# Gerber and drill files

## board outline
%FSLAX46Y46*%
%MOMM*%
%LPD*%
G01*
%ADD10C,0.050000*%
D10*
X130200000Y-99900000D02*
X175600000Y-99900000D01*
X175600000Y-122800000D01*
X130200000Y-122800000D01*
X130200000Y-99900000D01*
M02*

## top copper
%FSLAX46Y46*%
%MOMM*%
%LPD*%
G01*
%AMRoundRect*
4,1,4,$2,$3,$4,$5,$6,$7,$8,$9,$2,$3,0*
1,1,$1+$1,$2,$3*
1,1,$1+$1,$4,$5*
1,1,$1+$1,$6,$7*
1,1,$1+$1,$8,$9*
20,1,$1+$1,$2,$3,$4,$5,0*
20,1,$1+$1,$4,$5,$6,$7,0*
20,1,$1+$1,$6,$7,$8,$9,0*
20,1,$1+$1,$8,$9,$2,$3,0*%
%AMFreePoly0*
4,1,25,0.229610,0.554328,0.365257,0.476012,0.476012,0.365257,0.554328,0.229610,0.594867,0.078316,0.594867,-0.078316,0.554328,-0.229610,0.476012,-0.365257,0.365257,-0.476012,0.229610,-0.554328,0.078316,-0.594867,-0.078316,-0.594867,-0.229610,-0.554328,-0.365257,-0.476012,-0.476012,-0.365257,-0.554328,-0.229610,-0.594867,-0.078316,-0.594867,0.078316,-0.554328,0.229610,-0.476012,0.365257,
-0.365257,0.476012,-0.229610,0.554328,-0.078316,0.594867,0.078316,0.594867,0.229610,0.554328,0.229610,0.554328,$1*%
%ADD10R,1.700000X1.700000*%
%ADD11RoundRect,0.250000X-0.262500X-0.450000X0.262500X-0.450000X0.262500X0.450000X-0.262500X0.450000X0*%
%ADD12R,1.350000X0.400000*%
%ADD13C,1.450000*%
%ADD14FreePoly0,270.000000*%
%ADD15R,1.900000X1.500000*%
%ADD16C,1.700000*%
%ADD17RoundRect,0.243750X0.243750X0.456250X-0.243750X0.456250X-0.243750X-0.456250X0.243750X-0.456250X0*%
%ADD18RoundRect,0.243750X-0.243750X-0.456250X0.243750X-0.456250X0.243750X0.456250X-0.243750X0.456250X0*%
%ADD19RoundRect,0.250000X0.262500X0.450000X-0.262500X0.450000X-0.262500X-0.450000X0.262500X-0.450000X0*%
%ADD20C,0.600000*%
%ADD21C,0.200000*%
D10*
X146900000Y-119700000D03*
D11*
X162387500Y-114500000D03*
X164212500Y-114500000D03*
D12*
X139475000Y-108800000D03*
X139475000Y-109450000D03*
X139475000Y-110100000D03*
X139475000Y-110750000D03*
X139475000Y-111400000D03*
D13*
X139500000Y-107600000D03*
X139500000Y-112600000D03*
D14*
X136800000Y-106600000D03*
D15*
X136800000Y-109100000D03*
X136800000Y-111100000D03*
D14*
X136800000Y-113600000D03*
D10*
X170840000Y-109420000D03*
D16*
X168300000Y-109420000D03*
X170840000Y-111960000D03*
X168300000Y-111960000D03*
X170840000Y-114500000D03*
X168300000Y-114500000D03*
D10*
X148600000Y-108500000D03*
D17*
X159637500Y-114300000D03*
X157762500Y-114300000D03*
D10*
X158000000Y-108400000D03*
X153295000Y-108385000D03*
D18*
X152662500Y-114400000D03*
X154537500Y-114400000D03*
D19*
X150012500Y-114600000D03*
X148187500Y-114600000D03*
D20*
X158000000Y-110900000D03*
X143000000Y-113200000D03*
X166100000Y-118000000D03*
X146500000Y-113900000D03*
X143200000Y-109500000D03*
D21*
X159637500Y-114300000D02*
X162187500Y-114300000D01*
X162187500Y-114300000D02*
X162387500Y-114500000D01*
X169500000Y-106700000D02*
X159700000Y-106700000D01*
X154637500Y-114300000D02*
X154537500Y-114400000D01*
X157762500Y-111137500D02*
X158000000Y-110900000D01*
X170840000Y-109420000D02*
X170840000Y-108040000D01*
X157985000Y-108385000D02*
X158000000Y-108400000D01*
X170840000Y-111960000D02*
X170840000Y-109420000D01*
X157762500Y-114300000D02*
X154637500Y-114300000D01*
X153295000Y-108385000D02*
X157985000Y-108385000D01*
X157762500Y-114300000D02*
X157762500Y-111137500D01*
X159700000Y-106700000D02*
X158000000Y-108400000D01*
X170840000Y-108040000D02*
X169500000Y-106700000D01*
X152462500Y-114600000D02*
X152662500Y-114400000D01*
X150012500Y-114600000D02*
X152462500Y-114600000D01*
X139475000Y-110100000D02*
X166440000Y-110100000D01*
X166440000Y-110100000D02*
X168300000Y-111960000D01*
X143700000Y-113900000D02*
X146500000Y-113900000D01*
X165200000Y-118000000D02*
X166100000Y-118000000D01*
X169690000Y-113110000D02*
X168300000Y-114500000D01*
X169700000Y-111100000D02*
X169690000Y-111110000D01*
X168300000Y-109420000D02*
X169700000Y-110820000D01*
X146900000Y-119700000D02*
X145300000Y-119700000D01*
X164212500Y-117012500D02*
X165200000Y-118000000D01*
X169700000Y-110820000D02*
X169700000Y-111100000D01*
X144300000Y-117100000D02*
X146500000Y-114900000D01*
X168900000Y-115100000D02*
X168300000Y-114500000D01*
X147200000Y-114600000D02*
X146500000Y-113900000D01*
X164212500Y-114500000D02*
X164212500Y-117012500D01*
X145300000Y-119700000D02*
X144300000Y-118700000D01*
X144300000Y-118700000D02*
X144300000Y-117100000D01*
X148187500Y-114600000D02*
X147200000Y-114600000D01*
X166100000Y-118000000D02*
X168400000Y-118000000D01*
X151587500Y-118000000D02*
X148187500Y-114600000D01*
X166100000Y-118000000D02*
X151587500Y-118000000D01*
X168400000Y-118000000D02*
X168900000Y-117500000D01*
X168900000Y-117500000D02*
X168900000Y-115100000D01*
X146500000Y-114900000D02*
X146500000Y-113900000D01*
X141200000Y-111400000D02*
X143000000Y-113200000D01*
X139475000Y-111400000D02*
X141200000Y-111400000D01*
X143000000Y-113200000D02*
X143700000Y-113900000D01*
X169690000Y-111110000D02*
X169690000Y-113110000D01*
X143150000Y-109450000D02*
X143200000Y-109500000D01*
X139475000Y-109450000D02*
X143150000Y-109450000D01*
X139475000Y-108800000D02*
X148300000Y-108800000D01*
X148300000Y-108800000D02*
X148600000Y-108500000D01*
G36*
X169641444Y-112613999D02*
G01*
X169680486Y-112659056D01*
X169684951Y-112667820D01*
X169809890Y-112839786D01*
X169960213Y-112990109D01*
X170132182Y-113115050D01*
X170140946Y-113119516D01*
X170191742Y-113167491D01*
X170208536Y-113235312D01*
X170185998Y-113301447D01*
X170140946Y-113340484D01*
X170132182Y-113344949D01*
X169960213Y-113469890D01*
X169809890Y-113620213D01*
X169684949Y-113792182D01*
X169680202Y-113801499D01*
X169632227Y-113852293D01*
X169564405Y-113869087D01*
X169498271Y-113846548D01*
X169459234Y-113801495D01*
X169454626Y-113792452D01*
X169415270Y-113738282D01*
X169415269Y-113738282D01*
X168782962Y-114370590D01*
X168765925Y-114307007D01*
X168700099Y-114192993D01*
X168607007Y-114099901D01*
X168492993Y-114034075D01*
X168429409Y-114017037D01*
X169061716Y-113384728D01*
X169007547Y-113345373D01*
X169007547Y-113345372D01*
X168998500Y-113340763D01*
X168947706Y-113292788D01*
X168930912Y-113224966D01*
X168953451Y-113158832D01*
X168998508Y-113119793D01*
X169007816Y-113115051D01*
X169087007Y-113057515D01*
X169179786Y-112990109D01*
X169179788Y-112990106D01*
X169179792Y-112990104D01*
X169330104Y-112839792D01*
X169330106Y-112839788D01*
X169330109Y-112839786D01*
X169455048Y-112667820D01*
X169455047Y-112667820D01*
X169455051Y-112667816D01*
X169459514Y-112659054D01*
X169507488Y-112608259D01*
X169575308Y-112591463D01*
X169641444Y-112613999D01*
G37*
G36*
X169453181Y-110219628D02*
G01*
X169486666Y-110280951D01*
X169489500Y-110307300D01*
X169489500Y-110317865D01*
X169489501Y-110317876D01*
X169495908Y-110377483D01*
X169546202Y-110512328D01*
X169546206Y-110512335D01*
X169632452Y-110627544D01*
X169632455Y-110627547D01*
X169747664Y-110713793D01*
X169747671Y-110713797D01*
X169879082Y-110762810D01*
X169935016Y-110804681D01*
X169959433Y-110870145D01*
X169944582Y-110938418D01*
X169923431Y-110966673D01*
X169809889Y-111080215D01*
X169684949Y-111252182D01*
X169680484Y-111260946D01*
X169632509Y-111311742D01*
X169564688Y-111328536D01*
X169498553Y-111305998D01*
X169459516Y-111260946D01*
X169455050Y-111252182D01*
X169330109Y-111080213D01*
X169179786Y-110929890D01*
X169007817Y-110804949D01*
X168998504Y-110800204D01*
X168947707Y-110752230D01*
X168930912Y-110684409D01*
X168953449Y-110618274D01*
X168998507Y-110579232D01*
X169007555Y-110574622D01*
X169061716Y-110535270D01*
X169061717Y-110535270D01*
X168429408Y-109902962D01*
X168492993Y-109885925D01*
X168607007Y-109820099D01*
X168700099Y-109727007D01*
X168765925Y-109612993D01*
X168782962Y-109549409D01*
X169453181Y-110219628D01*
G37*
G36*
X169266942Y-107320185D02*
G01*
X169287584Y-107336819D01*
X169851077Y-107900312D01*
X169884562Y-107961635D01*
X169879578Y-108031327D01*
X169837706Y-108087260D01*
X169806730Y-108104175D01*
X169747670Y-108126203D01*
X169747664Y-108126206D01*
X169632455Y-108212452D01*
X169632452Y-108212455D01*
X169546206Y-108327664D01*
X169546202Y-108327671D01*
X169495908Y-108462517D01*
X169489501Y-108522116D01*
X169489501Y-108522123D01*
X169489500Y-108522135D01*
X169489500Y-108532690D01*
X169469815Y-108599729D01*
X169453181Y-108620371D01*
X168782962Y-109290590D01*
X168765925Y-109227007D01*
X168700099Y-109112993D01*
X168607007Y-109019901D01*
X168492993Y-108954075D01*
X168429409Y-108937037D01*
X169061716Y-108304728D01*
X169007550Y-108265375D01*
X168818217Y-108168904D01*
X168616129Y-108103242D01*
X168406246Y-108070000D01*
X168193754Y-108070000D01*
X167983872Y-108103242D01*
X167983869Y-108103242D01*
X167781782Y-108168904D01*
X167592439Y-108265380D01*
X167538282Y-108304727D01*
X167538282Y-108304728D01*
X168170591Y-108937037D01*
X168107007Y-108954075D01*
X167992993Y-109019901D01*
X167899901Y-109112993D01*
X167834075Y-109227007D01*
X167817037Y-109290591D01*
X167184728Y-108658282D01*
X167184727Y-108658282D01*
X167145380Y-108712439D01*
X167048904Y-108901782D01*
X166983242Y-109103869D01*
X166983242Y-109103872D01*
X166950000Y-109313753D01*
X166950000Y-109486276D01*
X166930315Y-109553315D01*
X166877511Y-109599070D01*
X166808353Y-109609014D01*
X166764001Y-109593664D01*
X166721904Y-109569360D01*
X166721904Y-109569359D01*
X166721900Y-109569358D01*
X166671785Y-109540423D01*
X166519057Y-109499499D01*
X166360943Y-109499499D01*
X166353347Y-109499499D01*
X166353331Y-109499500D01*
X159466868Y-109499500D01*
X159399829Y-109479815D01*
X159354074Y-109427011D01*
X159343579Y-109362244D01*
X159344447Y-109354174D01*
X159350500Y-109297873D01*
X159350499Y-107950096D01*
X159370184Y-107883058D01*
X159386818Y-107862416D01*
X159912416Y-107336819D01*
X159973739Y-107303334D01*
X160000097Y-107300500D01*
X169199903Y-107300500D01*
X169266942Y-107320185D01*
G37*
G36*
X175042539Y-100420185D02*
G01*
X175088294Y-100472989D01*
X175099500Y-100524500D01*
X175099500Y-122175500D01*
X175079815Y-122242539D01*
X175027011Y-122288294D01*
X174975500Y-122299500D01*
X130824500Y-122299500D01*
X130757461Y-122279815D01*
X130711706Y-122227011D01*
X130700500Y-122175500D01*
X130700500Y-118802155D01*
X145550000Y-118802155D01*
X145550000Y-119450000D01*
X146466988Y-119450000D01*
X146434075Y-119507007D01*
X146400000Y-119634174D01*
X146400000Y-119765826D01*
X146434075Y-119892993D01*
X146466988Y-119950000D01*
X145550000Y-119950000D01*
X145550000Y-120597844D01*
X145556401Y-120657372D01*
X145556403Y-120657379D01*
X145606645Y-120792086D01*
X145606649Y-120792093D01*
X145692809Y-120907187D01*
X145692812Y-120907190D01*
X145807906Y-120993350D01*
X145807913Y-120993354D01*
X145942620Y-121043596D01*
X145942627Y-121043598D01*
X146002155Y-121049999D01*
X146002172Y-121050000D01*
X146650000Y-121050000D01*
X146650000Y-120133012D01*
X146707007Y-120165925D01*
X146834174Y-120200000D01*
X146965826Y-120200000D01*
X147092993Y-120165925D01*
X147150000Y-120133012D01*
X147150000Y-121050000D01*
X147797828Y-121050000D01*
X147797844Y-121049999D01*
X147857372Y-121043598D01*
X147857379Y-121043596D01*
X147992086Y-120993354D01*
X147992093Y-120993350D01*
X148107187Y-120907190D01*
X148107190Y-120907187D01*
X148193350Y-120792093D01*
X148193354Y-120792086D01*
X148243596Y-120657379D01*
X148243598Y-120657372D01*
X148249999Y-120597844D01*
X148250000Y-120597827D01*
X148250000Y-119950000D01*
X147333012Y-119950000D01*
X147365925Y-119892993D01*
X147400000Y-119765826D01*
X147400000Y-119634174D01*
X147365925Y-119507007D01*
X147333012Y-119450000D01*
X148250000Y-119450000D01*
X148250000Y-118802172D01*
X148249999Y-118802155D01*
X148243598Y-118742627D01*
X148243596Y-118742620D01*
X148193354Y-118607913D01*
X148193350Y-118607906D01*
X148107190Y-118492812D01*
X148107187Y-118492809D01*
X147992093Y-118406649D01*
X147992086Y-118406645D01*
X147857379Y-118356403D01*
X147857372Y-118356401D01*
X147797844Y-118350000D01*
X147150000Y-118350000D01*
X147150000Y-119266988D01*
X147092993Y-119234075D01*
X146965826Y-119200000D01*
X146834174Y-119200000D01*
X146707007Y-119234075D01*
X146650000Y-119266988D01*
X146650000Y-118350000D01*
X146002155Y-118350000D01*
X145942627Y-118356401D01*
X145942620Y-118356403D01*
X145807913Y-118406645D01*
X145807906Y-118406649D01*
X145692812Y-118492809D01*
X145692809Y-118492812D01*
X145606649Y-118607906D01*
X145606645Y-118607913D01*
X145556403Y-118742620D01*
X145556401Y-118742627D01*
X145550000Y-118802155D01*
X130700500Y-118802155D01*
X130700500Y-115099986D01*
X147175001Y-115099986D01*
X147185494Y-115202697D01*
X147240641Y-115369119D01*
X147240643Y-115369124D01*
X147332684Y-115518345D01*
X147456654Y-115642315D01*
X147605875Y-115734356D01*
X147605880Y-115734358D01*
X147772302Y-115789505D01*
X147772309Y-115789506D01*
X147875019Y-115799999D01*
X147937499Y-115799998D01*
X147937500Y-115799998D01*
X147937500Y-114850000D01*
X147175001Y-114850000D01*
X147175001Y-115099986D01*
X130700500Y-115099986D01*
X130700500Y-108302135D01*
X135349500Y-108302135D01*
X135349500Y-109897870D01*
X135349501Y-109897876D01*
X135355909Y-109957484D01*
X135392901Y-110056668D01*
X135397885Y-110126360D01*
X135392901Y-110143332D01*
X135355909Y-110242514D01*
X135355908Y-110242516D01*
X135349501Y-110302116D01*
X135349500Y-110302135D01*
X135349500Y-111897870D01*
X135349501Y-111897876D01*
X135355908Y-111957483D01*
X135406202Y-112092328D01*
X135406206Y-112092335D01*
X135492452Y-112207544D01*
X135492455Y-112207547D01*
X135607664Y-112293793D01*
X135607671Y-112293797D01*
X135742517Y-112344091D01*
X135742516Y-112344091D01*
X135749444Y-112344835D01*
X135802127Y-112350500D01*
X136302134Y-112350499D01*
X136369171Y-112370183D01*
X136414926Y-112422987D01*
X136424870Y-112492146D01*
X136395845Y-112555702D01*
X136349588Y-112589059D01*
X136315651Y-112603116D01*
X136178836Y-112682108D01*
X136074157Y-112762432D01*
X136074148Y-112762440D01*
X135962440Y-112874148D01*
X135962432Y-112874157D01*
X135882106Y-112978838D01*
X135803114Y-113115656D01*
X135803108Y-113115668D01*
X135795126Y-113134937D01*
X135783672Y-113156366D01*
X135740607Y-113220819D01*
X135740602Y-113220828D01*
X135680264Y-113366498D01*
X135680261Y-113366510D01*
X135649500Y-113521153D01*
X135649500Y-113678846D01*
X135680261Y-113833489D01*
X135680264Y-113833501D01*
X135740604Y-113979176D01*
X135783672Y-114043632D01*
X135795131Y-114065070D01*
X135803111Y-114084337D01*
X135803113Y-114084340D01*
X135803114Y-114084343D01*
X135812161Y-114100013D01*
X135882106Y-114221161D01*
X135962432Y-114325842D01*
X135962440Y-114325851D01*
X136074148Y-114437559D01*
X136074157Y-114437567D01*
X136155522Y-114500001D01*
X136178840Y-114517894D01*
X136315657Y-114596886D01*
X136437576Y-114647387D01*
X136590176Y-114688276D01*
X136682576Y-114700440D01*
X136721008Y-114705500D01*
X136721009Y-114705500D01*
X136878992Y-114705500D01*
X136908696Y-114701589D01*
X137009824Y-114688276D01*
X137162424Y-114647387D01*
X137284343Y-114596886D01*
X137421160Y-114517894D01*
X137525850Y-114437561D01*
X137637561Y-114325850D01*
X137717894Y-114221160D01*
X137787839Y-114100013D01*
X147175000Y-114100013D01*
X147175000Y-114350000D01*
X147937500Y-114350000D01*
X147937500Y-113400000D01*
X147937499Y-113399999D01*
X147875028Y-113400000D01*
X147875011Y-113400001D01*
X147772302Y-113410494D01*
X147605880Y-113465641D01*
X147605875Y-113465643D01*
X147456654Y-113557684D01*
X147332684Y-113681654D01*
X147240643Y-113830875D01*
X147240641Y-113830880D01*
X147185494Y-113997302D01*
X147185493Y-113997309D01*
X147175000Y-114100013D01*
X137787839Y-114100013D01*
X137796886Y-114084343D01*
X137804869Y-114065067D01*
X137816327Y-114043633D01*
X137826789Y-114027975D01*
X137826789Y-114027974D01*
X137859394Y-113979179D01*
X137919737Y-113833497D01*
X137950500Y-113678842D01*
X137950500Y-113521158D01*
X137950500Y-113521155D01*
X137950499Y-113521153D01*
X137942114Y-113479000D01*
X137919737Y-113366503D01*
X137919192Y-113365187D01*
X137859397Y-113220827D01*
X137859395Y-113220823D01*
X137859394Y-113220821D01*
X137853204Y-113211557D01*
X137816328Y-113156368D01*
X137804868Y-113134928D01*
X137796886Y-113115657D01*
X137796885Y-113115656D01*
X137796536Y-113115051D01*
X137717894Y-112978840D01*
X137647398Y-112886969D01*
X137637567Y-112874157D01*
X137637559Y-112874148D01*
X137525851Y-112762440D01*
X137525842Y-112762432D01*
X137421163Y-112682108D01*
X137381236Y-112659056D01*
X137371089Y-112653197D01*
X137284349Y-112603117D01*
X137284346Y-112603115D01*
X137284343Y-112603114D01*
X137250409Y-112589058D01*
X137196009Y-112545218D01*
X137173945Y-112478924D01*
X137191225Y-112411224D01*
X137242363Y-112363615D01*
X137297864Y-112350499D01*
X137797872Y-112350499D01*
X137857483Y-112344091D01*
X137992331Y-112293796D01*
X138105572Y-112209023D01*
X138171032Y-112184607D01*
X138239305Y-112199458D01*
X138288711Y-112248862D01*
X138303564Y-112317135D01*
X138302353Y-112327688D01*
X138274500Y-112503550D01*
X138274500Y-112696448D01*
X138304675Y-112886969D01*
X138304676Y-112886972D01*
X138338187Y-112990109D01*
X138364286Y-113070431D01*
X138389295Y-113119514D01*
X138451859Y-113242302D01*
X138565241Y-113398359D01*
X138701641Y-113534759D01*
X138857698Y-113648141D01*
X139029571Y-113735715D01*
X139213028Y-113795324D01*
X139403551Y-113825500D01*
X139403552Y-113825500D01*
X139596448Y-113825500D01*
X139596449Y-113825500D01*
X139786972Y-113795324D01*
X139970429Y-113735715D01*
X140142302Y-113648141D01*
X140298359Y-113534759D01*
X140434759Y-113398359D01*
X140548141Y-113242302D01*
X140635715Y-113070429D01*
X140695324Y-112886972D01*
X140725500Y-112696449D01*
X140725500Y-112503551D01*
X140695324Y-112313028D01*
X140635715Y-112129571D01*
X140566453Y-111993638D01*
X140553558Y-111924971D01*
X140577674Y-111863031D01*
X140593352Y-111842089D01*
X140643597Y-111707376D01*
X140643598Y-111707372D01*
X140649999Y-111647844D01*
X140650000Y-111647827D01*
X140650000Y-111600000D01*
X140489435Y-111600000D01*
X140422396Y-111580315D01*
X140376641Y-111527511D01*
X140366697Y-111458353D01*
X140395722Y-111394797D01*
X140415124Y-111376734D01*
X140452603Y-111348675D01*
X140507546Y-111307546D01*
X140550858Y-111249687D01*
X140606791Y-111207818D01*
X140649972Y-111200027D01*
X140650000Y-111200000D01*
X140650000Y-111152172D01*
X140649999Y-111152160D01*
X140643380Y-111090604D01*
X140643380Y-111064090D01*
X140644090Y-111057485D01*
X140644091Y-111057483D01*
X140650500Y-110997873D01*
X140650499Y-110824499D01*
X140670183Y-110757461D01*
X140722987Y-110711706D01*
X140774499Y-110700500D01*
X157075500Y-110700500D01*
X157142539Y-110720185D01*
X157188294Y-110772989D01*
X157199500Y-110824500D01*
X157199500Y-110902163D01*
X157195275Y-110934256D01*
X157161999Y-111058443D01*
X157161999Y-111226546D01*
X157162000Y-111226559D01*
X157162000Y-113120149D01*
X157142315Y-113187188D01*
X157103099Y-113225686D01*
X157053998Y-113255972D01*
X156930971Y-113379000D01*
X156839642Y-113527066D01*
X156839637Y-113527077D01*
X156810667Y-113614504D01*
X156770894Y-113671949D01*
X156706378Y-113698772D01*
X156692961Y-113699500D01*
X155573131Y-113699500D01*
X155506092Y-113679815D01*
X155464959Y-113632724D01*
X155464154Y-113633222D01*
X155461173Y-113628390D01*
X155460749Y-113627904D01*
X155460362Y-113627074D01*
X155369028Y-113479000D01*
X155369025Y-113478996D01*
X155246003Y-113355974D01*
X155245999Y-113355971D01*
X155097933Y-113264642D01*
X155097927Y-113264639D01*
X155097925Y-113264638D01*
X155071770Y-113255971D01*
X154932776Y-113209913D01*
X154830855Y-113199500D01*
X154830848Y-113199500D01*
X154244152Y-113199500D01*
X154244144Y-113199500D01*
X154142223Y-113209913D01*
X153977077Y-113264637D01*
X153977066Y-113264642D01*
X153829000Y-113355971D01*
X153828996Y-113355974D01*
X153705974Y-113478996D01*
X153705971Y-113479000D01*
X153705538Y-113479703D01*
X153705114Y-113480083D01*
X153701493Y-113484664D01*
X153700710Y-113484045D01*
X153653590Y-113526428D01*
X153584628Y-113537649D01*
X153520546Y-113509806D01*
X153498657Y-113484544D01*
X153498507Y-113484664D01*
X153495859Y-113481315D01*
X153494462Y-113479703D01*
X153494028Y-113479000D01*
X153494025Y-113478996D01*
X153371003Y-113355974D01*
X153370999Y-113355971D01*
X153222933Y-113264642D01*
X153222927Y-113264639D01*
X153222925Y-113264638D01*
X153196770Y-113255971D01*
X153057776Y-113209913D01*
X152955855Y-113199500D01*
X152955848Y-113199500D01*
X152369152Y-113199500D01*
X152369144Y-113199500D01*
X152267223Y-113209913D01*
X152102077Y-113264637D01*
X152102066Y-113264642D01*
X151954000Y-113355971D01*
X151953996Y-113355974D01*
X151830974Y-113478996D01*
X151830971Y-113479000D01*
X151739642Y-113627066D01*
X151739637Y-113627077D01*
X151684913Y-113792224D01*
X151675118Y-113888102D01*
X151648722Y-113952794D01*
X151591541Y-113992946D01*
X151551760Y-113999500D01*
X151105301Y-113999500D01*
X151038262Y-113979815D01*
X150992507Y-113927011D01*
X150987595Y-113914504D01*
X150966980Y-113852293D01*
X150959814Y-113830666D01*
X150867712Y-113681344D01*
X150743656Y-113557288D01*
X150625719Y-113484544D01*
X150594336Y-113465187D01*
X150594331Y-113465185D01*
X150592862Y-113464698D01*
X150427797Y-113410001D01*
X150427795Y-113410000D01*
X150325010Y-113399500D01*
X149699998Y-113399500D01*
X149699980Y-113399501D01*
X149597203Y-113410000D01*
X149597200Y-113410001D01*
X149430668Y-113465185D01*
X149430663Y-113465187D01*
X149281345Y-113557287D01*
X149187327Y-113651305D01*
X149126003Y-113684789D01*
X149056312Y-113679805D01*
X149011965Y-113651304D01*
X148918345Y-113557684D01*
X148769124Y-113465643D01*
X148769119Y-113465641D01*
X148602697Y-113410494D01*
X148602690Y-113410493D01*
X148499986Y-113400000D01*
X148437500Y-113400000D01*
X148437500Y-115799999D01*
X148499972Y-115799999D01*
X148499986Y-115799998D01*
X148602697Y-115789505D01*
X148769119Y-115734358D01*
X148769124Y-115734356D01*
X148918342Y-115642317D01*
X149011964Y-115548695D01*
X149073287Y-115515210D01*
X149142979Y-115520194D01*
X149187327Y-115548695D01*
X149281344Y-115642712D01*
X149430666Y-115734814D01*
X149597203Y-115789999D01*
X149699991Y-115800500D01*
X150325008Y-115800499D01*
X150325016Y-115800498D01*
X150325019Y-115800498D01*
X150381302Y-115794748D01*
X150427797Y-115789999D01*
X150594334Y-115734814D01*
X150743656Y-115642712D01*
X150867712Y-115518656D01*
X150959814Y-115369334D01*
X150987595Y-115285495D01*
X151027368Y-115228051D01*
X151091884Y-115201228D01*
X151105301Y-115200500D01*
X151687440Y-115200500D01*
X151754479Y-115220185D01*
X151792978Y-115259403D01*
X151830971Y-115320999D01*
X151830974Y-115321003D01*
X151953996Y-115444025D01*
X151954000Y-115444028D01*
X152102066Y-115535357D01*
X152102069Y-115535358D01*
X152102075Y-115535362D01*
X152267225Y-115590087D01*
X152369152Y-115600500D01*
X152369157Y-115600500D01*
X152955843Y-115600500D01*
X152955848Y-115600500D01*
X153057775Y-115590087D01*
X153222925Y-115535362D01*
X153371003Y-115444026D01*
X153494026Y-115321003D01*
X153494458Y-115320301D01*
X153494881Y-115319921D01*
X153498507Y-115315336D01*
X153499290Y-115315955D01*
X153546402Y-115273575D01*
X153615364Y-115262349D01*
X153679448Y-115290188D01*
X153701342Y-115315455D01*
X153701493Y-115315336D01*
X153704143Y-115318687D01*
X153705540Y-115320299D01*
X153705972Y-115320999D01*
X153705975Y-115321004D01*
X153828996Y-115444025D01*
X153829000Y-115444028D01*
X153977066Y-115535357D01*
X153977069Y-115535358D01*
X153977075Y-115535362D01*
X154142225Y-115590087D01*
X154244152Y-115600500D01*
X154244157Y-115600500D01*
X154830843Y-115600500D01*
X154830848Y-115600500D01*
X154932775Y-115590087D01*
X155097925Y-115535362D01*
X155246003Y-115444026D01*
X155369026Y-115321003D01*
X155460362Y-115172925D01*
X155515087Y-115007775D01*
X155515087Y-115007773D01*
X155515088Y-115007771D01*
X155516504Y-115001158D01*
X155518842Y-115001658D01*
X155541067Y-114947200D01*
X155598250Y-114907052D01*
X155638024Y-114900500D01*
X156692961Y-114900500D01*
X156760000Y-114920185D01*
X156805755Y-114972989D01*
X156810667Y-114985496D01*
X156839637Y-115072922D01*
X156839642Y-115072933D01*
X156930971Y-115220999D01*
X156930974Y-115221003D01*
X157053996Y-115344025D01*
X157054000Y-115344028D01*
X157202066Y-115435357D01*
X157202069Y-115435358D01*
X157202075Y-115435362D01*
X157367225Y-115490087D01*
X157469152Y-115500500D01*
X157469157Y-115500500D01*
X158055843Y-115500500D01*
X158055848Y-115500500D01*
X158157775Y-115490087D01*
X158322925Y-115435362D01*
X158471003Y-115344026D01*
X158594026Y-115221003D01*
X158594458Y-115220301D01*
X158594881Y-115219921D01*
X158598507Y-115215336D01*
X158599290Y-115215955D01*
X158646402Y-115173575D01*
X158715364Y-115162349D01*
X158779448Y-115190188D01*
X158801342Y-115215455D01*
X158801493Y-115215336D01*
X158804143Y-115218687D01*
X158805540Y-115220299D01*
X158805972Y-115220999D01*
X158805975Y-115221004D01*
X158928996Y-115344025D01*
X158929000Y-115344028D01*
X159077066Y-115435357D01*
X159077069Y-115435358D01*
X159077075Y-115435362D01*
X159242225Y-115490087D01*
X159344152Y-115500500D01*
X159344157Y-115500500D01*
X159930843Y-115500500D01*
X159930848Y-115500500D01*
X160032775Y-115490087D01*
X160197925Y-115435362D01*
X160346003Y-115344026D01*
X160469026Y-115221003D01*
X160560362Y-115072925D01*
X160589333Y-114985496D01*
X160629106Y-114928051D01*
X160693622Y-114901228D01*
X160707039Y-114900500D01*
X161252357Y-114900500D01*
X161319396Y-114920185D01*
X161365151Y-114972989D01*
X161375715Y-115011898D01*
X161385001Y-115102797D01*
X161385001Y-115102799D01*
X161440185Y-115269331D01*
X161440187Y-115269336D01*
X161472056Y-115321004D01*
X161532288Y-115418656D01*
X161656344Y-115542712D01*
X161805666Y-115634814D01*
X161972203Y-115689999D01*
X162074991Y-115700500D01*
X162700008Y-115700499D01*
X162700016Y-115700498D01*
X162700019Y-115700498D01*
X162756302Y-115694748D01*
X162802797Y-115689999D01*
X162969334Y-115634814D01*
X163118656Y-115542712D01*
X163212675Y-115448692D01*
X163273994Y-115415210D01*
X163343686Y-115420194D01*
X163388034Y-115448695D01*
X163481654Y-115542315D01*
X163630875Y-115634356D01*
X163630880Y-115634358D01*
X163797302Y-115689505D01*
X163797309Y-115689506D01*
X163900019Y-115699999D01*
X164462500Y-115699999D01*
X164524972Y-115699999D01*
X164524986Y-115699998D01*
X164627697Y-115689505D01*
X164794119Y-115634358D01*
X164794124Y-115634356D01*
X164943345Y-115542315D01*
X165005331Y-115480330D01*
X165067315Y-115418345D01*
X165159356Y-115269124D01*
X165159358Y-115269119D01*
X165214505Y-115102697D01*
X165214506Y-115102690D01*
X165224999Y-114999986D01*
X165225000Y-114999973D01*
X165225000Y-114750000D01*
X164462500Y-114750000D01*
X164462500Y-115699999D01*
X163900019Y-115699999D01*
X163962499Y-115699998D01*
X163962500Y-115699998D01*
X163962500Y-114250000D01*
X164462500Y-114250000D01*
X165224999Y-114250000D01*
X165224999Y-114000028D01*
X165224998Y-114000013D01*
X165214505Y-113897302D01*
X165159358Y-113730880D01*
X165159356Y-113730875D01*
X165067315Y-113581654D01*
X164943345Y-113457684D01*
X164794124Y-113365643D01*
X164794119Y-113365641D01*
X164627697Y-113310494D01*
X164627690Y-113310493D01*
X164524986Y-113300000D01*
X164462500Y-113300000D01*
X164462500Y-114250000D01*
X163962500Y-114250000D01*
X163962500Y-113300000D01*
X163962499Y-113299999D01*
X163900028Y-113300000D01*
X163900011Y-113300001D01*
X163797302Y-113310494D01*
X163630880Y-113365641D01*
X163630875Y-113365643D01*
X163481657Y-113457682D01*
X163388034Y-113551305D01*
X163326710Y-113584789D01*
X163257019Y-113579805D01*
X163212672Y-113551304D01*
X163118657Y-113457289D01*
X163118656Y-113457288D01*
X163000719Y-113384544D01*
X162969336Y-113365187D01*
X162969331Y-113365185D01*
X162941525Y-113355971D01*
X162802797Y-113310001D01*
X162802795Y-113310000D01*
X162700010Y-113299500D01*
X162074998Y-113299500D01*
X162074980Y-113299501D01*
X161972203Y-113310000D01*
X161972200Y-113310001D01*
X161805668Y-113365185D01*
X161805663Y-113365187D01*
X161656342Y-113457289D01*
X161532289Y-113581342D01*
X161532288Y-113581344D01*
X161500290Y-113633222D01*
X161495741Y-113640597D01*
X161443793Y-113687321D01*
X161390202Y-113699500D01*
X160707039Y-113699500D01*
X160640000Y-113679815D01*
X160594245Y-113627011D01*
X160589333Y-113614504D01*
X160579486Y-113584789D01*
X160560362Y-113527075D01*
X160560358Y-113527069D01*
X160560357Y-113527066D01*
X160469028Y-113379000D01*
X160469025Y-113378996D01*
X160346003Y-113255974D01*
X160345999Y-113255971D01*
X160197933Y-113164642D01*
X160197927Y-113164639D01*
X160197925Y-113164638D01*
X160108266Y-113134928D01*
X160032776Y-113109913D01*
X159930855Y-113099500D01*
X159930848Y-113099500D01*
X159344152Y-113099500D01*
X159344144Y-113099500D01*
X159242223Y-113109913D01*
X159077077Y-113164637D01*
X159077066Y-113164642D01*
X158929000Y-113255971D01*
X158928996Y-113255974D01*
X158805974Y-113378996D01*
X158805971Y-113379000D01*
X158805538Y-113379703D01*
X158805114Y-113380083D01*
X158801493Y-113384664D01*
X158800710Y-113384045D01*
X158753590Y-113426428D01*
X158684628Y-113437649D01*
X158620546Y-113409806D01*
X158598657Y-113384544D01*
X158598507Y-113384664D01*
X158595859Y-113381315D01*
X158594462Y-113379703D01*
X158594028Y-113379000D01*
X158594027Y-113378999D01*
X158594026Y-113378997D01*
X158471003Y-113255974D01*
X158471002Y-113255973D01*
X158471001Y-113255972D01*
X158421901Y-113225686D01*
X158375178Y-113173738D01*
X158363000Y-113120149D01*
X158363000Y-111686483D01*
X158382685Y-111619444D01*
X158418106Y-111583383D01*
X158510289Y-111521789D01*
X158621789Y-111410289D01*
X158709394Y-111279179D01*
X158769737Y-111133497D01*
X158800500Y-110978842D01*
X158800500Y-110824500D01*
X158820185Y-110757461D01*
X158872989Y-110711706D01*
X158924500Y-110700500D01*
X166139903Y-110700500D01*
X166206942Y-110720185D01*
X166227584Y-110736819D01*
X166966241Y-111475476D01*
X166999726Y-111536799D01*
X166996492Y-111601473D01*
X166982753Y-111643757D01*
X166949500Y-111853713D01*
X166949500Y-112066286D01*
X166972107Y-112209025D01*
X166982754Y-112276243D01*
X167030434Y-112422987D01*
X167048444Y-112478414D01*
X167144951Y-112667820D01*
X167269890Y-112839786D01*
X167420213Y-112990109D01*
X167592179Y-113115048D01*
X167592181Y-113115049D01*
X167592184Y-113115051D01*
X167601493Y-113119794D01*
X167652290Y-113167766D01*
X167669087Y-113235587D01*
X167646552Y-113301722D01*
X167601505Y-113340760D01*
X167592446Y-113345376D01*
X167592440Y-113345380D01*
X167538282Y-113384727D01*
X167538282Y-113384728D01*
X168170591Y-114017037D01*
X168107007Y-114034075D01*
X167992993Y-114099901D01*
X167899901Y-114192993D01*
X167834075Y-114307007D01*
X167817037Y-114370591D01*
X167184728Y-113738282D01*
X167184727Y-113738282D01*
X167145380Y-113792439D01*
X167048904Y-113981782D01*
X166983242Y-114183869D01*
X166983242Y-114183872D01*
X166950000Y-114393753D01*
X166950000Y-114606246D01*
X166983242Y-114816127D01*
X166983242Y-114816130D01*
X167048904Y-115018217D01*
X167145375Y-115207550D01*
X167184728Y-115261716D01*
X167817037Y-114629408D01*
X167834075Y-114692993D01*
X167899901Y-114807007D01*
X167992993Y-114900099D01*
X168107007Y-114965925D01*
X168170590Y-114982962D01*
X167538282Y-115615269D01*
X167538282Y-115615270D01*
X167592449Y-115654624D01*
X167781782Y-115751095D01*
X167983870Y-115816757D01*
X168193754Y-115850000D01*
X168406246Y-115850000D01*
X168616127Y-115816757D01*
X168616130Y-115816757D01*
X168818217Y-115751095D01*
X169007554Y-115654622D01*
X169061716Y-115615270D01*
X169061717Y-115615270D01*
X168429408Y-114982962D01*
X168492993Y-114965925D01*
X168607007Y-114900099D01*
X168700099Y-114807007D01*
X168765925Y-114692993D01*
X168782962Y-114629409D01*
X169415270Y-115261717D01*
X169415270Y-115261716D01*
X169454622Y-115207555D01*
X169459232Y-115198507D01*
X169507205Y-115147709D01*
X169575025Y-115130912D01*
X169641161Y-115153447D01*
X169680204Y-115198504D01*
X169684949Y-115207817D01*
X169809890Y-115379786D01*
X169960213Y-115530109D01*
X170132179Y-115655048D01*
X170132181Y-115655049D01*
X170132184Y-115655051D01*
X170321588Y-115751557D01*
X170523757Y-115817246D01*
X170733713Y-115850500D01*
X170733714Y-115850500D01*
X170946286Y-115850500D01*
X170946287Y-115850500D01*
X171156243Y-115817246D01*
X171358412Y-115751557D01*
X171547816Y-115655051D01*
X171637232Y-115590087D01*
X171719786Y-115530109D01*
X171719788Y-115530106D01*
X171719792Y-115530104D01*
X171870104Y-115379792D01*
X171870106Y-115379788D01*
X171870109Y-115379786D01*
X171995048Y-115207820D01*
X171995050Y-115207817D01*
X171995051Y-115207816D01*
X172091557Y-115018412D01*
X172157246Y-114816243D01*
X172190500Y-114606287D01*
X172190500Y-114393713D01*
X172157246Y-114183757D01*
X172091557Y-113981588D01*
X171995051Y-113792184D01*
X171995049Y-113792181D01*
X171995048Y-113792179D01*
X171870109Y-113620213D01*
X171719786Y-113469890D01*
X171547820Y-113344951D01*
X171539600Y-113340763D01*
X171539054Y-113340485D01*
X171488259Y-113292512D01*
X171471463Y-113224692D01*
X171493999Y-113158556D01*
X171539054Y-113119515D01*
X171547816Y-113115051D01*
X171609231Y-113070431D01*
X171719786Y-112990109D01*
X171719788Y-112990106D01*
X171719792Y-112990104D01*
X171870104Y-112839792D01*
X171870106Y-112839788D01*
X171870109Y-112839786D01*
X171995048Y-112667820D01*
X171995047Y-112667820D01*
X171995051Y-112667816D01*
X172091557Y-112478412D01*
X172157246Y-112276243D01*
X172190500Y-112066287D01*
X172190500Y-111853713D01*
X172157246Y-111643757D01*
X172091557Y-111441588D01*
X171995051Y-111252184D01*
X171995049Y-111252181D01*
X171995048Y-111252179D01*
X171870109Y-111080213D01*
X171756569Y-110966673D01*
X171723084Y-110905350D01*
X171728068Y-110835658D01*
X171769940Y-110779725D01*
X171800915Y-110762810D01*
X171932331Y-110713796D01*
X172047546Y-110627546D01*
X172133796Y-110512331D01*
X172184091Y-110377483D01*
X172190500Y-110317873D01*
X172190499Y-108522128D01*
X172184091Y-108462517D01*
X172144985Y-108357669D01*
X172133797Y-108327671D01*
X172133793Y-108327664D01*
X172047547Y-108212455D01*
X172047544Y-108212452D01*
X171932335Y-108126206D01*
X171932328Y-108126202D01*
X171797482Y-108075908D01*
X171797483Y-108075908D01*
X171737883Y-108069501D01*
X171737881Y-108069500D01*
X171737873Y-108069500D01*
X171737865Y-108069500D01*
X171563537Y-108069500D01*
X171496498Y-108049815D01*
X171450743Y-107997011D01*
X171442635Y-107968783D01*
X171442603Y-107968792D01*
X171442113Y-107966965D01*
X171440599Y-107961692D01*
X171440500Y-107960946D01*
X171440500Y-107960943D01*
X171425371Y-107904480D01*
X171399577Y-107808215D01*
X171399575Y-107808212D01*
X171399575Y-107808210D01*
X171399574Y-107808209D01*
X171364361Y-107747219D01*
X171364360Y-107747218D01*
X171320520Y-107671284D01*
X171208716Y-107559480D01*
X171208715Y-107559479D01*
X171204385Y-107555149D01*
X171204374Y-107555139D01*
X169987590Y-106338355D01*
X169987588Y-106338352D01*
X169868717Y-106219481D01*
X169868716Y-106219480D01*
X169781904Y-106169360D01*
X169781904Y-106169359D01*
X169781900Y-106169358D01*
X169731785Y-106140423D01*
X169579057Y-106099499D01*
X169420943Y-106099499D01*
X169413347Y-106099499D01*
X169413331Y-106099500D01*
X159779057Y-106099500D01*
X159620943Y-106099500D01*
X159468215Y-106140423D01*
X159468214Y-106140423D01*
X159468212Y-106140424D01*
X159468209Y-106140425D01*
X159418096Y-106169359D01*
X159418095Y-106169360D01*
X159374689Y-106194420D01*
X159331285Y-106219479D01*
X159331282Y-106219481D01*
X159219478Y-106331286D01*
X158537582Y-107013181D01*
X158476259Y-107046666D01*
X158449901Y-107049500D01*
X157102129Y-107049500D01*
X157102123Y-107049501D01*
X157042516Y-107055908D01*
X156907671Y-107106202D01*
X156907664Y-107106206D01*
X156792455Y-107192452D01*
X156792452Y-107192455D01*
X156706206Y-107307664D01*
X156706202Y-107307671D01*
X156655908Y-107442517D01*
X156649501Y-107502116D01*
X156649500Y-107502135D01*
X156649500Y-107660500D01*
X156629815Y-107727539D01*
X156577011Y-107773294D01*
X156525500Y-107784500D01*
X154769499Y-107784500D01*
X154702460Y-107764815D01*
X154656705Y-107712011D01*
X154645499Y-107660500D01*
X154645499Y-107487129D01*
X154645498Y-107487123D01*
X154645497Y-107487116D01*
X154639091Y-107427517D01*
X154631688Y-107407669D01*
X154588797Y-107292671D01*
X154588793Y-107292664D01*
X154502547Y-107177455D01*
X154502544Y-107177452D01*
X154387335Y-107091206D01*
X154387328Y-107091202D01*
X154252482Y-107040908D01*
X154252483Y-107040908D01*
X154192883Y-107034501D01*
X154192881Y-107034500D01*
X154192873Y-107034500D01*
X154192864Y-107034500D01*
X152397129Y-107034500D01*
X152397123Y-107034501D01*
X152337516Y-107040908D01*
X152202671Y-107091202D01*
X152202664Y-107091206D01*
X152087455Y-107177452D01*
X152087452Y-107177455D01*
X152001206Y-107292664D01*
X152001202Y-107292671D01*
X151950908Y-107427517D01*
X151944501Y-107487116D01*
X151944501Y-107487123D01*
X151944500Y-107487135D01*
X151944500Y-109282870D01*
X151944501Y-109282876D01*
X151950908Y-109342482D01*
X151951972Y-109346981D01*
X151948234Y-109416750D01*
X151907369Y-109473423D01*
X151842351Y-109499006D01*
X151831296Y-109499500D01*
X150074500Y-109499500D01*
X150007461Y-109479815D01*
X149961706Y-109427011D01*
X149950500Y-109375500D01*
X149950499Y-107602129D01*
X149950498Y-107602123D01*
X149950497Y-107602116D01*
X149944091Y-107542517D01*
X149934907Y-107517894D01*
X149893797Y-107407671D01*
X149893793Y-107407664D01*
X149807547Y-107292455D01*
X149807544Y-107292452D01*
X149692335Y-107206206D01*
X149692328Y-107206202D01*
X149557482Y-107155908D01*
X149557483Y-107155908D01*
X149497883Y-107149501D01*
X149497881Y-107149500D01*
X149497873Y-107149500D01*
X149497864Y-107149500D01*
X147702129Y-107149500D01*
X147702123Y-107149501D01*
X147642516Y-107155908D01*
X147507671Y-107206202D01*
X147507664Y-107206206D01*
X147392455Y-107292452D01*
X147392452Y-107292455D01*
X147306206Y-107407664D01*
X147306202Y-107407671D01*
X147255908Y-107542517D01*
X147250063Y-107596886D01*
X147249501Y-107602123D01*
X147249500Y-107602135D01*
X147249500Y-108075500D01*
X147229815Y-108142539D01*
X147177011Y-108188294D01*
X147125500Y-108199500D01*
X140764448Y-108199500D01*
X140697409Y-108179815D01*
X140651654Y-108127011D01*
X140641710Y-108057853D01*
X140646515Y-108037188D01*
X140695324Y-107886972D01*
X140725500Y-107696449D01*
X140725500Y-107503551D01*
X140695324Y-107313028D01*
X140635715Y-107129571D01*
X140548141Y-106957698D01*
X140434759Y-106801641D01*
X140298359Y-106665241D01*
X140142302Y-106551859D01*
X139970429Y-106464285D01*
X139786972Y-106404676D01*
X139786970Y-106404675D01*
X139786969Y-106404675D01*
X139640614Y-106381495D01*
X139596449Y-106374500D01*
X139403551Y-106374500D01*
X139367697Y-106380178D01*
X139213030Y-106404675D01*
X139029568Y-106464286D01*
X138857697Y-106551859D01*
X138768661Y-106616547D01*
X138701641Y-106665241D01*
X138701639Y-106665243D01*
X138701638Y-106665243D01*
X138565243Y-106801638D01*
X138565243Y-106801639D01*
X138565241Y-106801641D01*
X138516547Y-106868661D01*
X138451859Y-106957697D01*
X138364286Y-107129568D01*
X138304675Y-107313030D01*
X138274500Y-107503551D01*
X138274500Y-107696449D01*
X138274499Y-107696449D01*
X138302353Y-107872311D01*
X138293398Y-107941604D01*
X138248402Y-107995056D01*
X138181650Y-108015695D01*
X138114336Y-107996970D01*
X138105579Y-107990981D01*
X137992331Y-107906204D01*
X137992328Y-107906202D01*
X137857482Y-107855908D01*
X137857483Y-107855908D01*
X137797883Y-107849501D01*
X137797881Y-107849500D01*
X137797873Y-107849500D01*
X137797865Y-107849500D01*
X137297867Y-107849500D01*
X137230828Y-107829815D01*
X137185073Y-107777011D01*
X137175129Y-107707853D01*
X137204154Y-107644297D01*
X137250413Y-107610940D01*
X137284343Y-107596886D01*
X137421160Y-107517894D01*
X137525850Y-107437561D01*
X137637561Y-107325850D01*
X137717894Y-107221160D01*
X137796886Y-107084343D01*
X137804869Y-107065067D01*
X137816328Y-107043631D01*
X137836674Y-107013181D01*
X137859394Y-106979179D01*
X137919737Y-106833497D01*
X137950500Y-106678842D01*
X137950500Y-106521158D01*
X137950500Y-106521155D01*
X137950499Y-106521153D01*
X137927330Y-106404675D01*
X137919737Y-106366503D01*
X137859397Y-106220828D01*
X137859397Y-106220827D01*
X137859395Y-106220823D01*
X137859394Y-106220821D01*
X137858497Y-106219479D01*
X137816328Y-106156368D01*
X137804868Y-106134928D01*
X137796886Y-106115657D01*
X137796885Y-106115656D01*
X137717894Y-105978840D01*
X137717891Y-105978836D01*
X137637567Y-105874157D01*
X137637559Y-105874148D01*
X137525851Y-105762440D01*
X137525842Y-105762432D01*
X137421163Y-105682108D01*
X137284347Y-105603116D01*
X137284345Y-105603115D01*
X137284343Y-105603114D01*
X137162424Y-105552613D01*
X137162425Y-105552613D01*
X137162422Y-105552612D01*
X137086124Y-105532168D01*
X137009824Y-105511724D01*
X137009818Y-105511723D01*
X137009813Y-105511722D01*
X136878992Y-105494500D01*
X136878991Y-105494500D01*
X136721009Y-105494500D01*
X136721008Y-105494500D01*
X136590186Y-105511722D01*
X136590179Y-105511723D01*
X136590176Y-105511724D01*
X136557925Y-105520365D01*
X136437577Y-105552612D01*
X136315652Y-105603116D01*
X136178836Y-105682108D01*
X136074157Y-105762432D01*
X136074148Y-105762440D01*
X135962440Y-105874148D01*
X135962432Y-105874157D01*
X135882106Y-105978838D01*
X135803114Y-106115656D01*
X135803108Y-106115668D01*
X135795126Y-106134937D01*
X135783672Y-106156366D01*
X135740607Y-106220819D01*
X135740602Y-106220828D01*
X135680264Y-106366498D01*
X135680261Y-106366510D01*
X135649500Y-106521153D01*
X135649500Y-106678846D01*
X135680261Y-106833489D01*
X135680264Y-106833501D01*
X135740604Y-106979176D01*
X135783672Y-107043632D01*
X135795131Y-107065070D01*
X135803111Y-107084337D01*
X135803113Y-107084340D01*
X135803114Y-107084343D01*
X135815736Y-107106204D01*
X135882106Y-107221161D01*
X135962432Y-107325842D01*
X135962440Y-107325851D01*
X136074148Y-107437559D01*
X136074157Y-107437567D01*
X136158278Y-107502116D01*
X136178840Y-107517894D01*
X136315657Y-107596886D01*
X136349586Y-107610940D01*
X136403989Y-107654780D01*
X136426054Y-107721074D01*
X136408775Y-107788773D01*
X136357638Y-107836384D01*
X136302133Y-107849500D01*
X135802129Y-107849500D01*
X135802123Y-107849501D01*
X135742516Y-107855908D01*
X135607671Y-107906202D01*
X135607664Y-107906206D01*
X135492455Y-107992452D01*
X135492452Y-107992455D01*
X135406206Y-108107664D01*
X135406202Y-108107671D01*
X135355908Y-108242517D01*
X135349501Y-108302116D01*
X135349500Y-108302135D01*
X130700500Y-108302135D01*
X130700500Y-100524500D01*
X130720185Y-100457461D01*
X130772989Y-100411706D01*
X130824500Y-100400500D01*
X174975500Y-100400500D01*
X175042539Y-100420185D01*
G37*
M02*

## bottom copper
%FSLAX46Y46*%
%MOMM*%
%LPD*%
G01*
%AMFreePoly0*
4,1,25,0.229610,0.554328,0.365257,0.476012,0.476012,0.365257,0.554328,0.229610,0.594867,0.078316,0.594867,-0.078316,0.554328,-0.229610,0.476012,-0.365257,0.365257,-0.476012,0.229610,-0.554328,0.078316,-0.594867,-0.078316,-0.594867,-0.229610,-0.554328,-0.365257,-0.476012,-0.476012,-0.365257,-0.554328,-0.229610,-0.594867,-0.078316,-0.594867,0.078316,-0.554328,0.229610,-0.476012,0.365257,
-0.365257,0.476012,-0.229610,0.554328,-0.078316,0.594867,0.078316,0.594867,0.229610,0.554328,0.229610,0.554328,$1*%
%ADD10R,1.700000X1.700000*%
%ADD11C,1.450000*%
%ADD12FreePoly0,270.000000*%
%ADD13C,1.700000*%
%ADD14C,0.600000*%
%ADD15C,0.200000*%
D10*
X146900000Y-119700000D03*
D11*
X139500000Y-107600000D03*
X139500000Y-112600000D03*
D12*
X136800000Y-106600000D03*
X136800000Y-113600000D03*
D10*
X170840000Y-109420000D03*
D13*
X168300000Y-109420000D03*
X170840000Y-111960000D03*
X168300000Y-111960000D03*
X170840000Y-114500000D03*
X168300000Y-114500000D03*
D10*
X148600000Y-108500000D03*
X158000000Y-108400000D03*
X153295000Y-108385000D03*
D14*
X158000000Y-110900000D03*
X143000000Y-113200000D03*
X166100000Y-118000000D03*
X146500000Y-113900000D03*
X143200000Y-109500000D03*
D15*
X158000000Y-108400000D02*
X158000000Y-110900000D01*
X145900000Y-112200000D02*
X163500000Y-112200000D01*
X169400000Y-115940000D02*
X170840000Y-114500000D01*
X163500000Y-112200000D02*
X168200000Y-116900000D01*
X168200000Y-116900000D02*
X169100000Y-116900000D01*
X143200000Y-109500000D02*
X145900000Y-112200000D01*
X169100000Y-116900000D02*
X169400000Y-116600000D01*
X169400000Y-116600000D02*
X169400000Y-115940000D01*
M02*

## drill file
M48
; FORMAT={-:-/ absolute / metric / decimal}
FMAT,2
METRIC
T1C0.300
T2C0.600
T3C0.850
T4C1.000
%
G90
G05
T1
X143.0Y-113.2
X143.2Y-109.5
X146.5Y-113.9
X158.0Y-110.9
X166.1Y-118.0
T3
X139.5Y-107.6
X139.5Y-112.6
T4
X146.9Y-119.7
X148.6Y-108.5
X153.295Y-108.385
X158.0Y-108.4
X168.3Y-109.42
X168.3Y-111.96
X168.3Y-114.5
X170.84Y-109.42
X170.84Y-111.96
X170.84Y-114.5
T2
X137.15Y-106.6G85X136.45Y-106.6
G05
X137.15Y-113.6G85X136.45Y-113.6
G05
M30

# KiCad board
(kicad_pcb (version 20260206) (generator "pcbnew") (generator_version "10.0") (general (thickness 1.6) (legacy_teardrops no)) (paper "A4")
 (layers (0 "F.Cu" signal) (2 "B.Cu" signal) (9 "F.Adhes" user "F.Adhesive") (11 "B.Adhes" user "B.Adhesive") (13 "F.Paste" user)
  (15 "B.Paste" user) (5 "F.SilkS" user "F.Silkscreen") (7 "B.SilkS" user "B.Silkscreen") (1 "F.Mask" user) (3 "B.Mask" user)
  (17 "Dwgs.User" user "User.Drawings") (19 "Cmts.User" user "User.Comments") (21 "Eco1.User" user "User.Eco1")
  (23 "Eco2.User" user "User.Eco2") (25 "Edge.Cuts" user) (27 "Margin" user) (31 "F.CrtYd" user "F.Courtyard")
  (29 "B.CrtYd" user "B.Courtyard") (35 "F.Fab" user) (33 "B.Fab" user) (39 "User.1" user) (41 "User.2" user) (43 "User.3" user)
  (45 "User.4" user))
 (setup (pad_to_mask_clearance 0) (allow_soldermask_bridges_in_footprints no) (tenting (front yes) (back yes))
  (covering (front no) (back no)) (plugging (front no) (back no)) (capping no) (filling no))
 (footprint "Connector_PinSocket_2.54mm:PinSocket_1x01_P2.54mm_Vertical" (layer "F.Cu") (at 146.9 119.7)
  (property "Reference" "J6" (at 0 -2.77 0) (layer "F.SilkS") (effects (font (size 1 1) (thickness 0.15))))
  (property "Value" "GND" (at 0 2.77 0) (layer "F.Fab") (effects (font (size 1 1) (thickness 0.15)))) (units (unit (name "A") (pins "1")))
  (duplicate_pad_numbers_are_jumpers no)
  (pad "1" thru_hole rect (at 0 0) (size 1.7 1.7) (drill 1) (layers "*.Cu" "*.Mask") (remove_unused_layers no) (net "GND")))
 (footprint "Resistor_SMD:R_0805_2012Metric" (layer "F.Cu") (at 163.3 114.5)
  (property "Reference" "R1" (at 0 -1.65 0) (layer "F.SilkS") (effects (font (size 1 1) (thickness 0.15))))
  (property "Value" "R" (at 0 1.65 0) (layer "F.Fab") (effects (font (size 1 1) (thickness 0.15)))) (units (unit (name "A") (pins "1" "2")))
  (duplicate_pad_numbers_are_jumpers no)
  (pad "1" smd roundrect (at -0.9125 0) (size 1.025 1.4) (layers "F.Cu" "F.Mask" "F.Paste") (roundrect_rratio 0.243902) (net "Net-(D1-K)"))
  (pad "2" smd roundrect (at 0.9125 0) (size 1.025 1.4) (layers "F.Cu" "F.Mask" "F.Paste") (roundrect_rratio 0.243902) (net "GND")))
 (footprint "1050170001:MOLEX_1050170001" (layer "F.Cu") (at 135.35 110.1 -90)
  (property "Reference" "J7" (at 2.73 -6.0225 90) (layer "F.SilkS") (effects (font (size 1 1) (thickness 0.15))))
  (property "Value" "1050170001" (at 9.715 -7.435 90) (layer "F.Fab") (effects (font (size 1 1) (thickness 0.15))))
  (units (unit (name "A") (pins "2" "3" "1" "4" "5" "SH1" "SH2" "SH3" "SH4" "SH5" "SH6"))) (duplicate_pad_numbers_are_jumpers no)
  (pad "1" smd rect (at -1.3 -4.125 270) (size 0.4 1.35) (layers "F.Cu" "F.Paste") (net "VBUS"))
  (pad "2" smd rect (at -0.65 -4.125 270) (size 0.4 1.35) (layers "F.Cu" "F.Paste") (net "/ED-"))
  (pad "3" smd rect (at 0 -4.125 270) (size 0.4 1.35) (layers "F.Cu" "F.Paste") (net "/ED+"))
  (pad "4" smd rect (at 0.65 -4.125 270) (size 0.4 1.35) (layers "F.Cu" "F.Paste") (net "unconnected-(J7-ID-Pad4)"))
  (pad "5" smd rect (at 1.3 -4.125 270) (size 0.4 1.35) (layers "F.Cu" "F.Paste") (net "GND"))
  (pad "SH1" thru_hole circle (at -2.5 -4.15 270) (size 1.45 1.45) (drill 0.85) (layers "*.Cu") (remove_unused_layers no)
   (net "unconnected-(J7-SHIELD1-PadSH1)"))
  (pad "SH2" thru_hole circle (at 2.5 -4.15 270) (size 1.45 1.45) (drill 0.85) (layers "*.Cu") (remove_unused_layers no)
   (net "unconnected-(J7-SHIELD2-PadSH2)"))
  (pad "SH3" thru_hole custom (at -3.5 -1.45 270) (size 1.2 1.9) (drill oval 0.6 1.3) (layers "*.Cu") (remove_unused_layers no)
   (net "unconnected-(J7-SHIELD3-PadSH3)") (thermal_bridge_angle 90) (options (clearance outline) (anchor circle)) (primitives))
  (pad "SH4" smd rect (at -1 -1.45 270) (size 1.5 1.9) (layers "F.Cu" "F.Paste") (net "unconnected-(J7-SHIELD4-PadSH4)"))
  (pad "SH5" smd rect (at 1 -1.45 270) (size 1.5 1.9) (layers "F.Cu" "F.Paste") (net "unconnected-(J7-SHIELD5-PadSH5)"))
  (pad "SH6" thru_hole custom (at 3.5 -1.45 270) (size 1.2 1.9) (drill oval 0.6 1.3) (layers "*.Cu") (remove_unused_layers no)
   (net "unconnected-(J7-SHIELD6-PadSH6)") (thermal_bridge_angle 90) (options (clearance outline) (anchor circle)) (primitives)))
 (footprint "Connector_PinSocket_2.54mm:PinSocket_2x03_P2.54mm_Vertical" (layer "F.Cu") (at 170.84 109.42)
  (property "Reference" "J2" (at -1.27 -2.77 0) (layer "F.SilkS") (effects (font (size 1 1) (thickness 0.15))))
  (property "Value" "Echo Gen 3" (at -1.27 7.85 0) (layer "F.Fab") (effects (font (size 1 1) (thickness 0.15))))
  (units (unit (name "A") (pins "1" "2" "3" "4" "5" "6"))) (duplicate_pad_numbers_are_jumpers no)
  (pad "1" thru_hole rect (at 0 0) (size 1.7 1.7) (drill 1) (layers "*.Cu" "*.Mask") (remove_unused_layers no) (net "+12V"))
  (pad "2" thru_hole circle (at -2.54 0) (size 1.7 1.7) (drill 1) (layers "*.Cu" "*.Mask") (remove_unused_layers no) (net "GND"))
  (pad "3" thru_hole circle (at 0 2.54) (size 1.7 1.7) (drill 1) (layers "*.Cu" "*.Mask") (remove_unused_layers no) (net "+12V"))
  (pad "4" thru_hole circle (at -2.54 2.54) (size 1.7 1.7) (drill 1) (layers "*.Cu" "*.Mask") (remove_unused_layers no) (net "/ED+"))
  (pad "5" thru_hole circle (at 0 5.08) (size 1.7 1.7) (drill 1) (layers "*.Cu" "*.Mask") (remove_unused_layers no) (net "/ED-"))
  (pad "6" thru_hole circle (at -2.54 5.08) (size 1.7 1.7) (drill 1) (layers "*.Cu" "*.Mask") (remove_unused_layers no) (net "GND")))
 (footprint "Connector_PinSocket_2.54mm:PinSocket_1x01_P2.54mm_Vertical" (layer "F.Cu") (at 148.6 108.5)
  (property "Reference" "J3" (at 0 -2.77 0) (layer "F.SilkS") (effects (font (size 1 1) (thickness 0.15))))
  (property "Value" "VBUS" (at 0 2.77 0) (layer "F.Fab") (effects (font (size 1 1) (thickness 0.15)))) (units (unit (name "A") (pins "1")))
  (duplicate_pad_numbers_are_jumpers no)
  (pad "1" thru_hole rect (at 0 0) (size 1.7 1.7) (drill 1) (layers "*.Cu" "*.Mask") (remove_unused_layers no) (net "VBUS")))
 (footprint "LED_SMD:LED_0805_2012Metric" (layer "F.Cu") (at 158.7 114.3 180)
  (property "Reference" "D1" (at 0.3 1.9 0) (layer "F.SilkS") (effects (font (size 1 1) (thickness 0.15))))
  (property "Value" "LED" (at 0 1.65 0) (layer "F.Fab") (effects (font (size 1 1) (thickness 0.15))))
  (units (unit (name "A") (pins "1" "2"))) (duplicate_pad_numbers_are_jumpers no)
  (pad "1" smd roundrect (at -0.9375 0 180) (size 0.975 1.4) (layers "F.Cu" "F.Mask" "F.Paste") (roundrect_rratio 0.25) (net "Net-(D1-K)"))
  (pad "2" smd roundrect (at 0.9375 0 180) (size 0.975 1.4) (layers "F.Cu" "F.Mask" "F.Paste") (roundrect_rratio 0.25) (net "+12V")))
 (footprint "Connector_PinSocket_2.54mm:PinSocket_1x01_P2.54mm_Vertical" (layer "F.Cu") (at 158 108.4)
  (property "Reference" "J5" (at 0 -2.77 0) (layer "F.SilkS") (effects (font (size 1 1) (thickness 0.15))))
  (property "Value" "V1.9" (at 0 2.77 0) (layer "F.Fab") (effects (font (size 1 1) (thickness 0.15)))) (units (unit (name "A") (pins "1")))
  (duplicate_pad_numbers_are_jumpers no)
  (pad "1" thru_hole rect (at 0 0) (size 1.7 1.7) (drill 1) (layers "*.Cu" "*.Mask") (remove_unused_layers no) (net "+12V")))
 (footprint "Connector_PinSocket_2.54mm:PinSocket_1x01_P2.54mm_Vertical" (layer "F.Cu") (at 153.295 108.385)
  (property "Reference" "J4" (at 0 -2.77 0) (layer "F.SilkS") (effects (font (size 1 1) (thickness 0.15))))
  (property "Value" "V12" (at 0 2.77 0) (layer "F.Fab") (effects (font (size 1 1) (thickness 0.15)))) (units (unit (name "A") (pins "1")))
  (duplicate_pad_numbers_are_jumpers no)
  (pad "1" thru_hole rect (at 0 0) (size 1.7 1.7) (drill 1) (layers "*.Cu" "*.Mask") (remove_unused_layers no) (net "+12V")))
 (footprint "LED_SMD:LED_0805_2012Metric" (layer "F.Cu") (at 153.6 114.4)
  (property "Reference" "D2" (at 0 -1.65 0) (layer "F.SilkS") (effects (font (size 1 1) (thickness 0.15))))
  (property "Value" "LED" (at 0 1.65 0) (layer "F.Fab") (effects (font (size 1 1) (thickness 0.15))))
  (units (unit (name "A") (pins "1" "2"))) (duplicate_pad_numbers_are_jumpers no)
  (pad "1" smd roundrect (at -0.9375 0) (size 0.975 1.4) (layers "F.Cu" "F.Mask" "F.Paste") (roundrect_rratio 0.25) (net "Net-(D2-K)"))
  (pad "2" smd roundrect (at 0.9375 0) (size 0.975 1.4) (layers "F.Cu" "F.Mask" "F.Paste") (roundrect_rratio 0.25) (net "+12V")))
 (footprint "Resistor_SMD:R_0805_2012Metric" (layer "F.Cu") (at 149.1 114.6 180)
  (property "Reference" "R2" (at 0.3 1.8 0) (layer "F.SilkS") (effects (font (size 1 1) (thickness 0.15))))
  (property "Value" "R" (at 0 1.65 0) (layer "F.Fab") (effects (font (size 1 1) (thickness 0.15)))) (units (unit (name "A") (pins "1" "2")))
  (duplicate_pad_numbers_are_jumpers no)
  (pad "1" smd roundrect (at -0.9125 0 180) (size 1.025 1.4) (layers "F.Cu" "F.Mask" "F.Paste") (roundrect_rratio 0.243902)
   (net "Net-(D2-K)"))
  (pad "2" smd roundrect (at 0.9125 0 180) (size 1.025 1.4) (layers "F.Cu" "F.Mask" "F.Paste") (roundrect_rratio 0.243902) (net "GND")))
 (gr_rect (start 130.2 99.9) (end 175.6 122.8) (stroke (width 0.05) (type default)) (fill no) (layer "Edge.Cuts"))
 (segment (start 159.6375 114.3) (end 162.1875 114.3) (width 0.2) (layer "F.Cu") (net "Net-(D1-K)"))
 (segment (start 162.1875 114.3) (end 162.3875 114.5) (width 0.2) (layer "F.Cu") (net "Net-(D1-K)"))
 (segment (start 169.5 106.7) (end 159.7 106.7) (width 0.2) (layer "F.Cu") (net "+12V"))
 (segment (start 154.6375 114.3) (end 154.5375 114.4) (width 0.2) (layer "F.Cu") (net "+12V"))
 (segment (start 157.7625 111.1375) (end 158 110.9) (width 0.2) (layer "F.Cu") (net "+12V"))
 (segment (start 170.84 109.42) (end 170.84 108.04) (width 0.2) (layer "F.Cu") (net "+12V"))
 (segment (start 157.985 108.385) (end 158 108.4) (width 0.2) (layer "F.Cu") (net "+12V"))
 (segment (start 170.84 111.96) (end 170.84 109.42) (width 0.2) (layer "F.Cu") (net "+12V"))
 (segment (start 157.7625 114.3) (end 154.6375 114.3) (width 0.2) (layer "F.Cu") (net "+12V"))
 (segment (start 153.295 108.385) (end 157.985 108.385) (width 0.2) (layer "F.Cu") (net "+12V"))
 (segment (start 157.7625 114.3) (end 157.7625 111.1375) (width 0.2) (layer "F.Cu") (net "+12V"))
 (segment (start 159.7 106.7) (end 158 108.4) (width 0.2) (layer "F.Cu") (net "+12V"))
 (segment (start 170.84 108.04) (end 169.5 106.7) (width 0.2) (layer "F.Cu") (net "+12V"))
 (via (at 158 110.9) (size 0.6) (drill 0.3) (layers "F.Cu" "B.Cu") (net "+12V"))
 (segment (start 158 108.4) (end 158 110.9) (width 0.2) (layer "B.Cu") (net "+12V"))
 (segment (start 152.4625 114.6) (end 152.6625 114.4) (width 0.2) (layer "F.Cu") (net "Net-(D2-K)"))
 (segment (start 150.0125 114.6) (end 152.4625 114.6) (width 0.2) (layer "F.Cu") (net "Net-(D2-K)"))
 (segment (start 139.475 110.1) (end 166.44 110.1) (width 0.2) (layer "F.Cu") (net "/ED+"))
 (segment (start 166.44 110.1) (end 168.3 111.96) (width 0.2) (layer "F.Cu") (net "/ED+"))
 (segment (start 143.7 113.9) (end 146.5 113.9) (width 0.2) (layer "F.Cu") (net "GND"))
 (segment (start 165.2 118) (end 166.1 118) (width 0.2) (layer "F.Cu") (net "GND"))
 (segment (start 169.69 113.11) (end 168.3 114.5) (width 0.2) (layer "F.Cu") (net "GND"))
 (segment (start 169.7 111.1) (end 169.69 111.11) (width 0.2) (layer "F.Cu") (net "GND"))
 (segment (start 168.3 109.42) (end 169.7 110.82) (width 0.2) (layer "F.Cu") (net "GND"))
 (segment (start 146.9 119.7) (end 145.3 119.7) (width 0.2) (layer "F.Cu") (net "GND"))
 (segment (start 164.2125 117.0125) (end 165.2 118) (width 0.2) (layer "F.Cu") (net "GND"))
 (segment (start 169.7 110.82) (end 169.7 111.1) (width 0.2) (layer "F.Cu") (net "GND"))
 (segment (start 144.3 117.1) (end 146.5 114.9) (width 0.2) (layer "F.Cu") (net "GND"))
 (segment (start 168.9 115.1) (end 168.3 114.5) (width 0.2) (layer "F.Cu") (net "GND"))
 (segment (start 147.2 114.6) (end 146.5 113.9) (width 0.2) (layer "F.Cu") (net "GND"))
 (segment (start 164.2125 114.5) (end 164.2125 117.0125) (width 0.2) (layer "F.Cu") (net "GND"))
 (segment (start 145.3 119.7) (end 144.3 118.7) (width 0.2) (layer "F.Cu") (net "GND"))
 (segment (start 144.3 118.7) (end 144.3 117.1) (width 0.2) (layer "F.Cu") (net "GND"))
 (segment (start 148.1875 114.6) (end 147.2 114.6) (width 0.2) (layer "F.Cu") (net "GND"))
 (segment (start 166.1 118) (end 168.4 118) (width 0.2) (layer "F.Cu") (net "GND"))
 (segment (start 151.5875 118) (end 148.1875 114.6) (width 0.2) (layer "F.Cu") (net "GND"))
 (segment (start 166.1 118) (end 151.5875 118) (width 0.2) (layer "F.Cu") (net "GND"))
 (segment (start 168.4 118) (end 168.9 117.5) (width 0.2) (layer "F.Cu") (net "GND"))
 (segment (start 168.9 117.5) (end 168.9 115.1) (width 0.2) (layer "F.Cu") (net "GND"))
 (segment (start 146.5 114.9) (end 146.5 113.9) (width 0.2) (layer "F.Cu") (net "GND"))
 (segment (start 141.2 111.4) (end 143 113.2) (width 0.2) (layer "F.Cu") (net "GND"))
 (segment (start 139.475 111.4) (end 141.2 111.4) (width 0.2) (layer "F.Cu") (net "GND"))
 (segment (start 143 113.2) (end 143.7 113.9) (width 0.2) (layer "F.Cu") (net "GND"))
 (segment (start 169.69 111.11) (end 169.69 113.11) (width 0.2) (layer "F.Cu") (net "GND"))
 (via (at 143 113.2) (size 0.6) (drill 0.3) (layers "F.Cu" "B.Cu") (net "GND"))
 (via (at 166.1 118) (size 0.6) (drill 0.3) (layers "F.Cu" "B.Cu") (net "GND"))
 (via (at 146.5 113.9) (size 0.6) (drill 0.3) (layers "F.Cu" "B.Cu") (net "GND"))
 (segment (start 143.15 109.45) (end 143.2 109.5) (width 0.2) (layer "F.Cu") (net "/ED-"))
 (segment (start 139.475 109.45) (end 143.15 109.45) (width 0.2) (layer "F.Cu") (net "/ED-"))
 (via (at 143.2 109.5) (size 0.6) (drill 0.3) (layers "F.Cu" "B.Cu") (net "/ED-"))
 (segment (start 145.9 112.2) (end 163.5 112.2) (width 0.2) (layer "B.Cu") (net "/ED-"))
 (segment (start 169.4 115.94) (end 170.84 114.5) (width 0.2) (layer "B.Cu") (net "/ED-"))
 (segment (start 163.5 112.2) (end 168.2 116.9) (width 0.2) (layer "B.Cu") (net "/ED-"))
 (segment (start 168.2 116.9) (end 169.1 116.9) (width 0.2) (layer "B.Cu") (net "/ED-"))
 (segment (start 143.2 109.5) (end 145.9 112.2) (width 0.2) (layer "B.Cu") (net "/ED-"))
 (segment (start 169.1 116.9) (end 169.4 116.6) (width 0.2) (layer "B.Cu") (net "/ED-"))
 (segment (start 169.4 116.6) (end 169.4 115.94) (width 0.2) (layer "B.Cu") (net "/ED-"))
 (segment (start 139.475 108.8) (end 148.3 108.8) (width 0.2) (layer "F.Cu") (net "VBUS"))
 (segment (start 148.3 108.8) (end 148.6 108.5) (width 0.2) (layer "F.Cu") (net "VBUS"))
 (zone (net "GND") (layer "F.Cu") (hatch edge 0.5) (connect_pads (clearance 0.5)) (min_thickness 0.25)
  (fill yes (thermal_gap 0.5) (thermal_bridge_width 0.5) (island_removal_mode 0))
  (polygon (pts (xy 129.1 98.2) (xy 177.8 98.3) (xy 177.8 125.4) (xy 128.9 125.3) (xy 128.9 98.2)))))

